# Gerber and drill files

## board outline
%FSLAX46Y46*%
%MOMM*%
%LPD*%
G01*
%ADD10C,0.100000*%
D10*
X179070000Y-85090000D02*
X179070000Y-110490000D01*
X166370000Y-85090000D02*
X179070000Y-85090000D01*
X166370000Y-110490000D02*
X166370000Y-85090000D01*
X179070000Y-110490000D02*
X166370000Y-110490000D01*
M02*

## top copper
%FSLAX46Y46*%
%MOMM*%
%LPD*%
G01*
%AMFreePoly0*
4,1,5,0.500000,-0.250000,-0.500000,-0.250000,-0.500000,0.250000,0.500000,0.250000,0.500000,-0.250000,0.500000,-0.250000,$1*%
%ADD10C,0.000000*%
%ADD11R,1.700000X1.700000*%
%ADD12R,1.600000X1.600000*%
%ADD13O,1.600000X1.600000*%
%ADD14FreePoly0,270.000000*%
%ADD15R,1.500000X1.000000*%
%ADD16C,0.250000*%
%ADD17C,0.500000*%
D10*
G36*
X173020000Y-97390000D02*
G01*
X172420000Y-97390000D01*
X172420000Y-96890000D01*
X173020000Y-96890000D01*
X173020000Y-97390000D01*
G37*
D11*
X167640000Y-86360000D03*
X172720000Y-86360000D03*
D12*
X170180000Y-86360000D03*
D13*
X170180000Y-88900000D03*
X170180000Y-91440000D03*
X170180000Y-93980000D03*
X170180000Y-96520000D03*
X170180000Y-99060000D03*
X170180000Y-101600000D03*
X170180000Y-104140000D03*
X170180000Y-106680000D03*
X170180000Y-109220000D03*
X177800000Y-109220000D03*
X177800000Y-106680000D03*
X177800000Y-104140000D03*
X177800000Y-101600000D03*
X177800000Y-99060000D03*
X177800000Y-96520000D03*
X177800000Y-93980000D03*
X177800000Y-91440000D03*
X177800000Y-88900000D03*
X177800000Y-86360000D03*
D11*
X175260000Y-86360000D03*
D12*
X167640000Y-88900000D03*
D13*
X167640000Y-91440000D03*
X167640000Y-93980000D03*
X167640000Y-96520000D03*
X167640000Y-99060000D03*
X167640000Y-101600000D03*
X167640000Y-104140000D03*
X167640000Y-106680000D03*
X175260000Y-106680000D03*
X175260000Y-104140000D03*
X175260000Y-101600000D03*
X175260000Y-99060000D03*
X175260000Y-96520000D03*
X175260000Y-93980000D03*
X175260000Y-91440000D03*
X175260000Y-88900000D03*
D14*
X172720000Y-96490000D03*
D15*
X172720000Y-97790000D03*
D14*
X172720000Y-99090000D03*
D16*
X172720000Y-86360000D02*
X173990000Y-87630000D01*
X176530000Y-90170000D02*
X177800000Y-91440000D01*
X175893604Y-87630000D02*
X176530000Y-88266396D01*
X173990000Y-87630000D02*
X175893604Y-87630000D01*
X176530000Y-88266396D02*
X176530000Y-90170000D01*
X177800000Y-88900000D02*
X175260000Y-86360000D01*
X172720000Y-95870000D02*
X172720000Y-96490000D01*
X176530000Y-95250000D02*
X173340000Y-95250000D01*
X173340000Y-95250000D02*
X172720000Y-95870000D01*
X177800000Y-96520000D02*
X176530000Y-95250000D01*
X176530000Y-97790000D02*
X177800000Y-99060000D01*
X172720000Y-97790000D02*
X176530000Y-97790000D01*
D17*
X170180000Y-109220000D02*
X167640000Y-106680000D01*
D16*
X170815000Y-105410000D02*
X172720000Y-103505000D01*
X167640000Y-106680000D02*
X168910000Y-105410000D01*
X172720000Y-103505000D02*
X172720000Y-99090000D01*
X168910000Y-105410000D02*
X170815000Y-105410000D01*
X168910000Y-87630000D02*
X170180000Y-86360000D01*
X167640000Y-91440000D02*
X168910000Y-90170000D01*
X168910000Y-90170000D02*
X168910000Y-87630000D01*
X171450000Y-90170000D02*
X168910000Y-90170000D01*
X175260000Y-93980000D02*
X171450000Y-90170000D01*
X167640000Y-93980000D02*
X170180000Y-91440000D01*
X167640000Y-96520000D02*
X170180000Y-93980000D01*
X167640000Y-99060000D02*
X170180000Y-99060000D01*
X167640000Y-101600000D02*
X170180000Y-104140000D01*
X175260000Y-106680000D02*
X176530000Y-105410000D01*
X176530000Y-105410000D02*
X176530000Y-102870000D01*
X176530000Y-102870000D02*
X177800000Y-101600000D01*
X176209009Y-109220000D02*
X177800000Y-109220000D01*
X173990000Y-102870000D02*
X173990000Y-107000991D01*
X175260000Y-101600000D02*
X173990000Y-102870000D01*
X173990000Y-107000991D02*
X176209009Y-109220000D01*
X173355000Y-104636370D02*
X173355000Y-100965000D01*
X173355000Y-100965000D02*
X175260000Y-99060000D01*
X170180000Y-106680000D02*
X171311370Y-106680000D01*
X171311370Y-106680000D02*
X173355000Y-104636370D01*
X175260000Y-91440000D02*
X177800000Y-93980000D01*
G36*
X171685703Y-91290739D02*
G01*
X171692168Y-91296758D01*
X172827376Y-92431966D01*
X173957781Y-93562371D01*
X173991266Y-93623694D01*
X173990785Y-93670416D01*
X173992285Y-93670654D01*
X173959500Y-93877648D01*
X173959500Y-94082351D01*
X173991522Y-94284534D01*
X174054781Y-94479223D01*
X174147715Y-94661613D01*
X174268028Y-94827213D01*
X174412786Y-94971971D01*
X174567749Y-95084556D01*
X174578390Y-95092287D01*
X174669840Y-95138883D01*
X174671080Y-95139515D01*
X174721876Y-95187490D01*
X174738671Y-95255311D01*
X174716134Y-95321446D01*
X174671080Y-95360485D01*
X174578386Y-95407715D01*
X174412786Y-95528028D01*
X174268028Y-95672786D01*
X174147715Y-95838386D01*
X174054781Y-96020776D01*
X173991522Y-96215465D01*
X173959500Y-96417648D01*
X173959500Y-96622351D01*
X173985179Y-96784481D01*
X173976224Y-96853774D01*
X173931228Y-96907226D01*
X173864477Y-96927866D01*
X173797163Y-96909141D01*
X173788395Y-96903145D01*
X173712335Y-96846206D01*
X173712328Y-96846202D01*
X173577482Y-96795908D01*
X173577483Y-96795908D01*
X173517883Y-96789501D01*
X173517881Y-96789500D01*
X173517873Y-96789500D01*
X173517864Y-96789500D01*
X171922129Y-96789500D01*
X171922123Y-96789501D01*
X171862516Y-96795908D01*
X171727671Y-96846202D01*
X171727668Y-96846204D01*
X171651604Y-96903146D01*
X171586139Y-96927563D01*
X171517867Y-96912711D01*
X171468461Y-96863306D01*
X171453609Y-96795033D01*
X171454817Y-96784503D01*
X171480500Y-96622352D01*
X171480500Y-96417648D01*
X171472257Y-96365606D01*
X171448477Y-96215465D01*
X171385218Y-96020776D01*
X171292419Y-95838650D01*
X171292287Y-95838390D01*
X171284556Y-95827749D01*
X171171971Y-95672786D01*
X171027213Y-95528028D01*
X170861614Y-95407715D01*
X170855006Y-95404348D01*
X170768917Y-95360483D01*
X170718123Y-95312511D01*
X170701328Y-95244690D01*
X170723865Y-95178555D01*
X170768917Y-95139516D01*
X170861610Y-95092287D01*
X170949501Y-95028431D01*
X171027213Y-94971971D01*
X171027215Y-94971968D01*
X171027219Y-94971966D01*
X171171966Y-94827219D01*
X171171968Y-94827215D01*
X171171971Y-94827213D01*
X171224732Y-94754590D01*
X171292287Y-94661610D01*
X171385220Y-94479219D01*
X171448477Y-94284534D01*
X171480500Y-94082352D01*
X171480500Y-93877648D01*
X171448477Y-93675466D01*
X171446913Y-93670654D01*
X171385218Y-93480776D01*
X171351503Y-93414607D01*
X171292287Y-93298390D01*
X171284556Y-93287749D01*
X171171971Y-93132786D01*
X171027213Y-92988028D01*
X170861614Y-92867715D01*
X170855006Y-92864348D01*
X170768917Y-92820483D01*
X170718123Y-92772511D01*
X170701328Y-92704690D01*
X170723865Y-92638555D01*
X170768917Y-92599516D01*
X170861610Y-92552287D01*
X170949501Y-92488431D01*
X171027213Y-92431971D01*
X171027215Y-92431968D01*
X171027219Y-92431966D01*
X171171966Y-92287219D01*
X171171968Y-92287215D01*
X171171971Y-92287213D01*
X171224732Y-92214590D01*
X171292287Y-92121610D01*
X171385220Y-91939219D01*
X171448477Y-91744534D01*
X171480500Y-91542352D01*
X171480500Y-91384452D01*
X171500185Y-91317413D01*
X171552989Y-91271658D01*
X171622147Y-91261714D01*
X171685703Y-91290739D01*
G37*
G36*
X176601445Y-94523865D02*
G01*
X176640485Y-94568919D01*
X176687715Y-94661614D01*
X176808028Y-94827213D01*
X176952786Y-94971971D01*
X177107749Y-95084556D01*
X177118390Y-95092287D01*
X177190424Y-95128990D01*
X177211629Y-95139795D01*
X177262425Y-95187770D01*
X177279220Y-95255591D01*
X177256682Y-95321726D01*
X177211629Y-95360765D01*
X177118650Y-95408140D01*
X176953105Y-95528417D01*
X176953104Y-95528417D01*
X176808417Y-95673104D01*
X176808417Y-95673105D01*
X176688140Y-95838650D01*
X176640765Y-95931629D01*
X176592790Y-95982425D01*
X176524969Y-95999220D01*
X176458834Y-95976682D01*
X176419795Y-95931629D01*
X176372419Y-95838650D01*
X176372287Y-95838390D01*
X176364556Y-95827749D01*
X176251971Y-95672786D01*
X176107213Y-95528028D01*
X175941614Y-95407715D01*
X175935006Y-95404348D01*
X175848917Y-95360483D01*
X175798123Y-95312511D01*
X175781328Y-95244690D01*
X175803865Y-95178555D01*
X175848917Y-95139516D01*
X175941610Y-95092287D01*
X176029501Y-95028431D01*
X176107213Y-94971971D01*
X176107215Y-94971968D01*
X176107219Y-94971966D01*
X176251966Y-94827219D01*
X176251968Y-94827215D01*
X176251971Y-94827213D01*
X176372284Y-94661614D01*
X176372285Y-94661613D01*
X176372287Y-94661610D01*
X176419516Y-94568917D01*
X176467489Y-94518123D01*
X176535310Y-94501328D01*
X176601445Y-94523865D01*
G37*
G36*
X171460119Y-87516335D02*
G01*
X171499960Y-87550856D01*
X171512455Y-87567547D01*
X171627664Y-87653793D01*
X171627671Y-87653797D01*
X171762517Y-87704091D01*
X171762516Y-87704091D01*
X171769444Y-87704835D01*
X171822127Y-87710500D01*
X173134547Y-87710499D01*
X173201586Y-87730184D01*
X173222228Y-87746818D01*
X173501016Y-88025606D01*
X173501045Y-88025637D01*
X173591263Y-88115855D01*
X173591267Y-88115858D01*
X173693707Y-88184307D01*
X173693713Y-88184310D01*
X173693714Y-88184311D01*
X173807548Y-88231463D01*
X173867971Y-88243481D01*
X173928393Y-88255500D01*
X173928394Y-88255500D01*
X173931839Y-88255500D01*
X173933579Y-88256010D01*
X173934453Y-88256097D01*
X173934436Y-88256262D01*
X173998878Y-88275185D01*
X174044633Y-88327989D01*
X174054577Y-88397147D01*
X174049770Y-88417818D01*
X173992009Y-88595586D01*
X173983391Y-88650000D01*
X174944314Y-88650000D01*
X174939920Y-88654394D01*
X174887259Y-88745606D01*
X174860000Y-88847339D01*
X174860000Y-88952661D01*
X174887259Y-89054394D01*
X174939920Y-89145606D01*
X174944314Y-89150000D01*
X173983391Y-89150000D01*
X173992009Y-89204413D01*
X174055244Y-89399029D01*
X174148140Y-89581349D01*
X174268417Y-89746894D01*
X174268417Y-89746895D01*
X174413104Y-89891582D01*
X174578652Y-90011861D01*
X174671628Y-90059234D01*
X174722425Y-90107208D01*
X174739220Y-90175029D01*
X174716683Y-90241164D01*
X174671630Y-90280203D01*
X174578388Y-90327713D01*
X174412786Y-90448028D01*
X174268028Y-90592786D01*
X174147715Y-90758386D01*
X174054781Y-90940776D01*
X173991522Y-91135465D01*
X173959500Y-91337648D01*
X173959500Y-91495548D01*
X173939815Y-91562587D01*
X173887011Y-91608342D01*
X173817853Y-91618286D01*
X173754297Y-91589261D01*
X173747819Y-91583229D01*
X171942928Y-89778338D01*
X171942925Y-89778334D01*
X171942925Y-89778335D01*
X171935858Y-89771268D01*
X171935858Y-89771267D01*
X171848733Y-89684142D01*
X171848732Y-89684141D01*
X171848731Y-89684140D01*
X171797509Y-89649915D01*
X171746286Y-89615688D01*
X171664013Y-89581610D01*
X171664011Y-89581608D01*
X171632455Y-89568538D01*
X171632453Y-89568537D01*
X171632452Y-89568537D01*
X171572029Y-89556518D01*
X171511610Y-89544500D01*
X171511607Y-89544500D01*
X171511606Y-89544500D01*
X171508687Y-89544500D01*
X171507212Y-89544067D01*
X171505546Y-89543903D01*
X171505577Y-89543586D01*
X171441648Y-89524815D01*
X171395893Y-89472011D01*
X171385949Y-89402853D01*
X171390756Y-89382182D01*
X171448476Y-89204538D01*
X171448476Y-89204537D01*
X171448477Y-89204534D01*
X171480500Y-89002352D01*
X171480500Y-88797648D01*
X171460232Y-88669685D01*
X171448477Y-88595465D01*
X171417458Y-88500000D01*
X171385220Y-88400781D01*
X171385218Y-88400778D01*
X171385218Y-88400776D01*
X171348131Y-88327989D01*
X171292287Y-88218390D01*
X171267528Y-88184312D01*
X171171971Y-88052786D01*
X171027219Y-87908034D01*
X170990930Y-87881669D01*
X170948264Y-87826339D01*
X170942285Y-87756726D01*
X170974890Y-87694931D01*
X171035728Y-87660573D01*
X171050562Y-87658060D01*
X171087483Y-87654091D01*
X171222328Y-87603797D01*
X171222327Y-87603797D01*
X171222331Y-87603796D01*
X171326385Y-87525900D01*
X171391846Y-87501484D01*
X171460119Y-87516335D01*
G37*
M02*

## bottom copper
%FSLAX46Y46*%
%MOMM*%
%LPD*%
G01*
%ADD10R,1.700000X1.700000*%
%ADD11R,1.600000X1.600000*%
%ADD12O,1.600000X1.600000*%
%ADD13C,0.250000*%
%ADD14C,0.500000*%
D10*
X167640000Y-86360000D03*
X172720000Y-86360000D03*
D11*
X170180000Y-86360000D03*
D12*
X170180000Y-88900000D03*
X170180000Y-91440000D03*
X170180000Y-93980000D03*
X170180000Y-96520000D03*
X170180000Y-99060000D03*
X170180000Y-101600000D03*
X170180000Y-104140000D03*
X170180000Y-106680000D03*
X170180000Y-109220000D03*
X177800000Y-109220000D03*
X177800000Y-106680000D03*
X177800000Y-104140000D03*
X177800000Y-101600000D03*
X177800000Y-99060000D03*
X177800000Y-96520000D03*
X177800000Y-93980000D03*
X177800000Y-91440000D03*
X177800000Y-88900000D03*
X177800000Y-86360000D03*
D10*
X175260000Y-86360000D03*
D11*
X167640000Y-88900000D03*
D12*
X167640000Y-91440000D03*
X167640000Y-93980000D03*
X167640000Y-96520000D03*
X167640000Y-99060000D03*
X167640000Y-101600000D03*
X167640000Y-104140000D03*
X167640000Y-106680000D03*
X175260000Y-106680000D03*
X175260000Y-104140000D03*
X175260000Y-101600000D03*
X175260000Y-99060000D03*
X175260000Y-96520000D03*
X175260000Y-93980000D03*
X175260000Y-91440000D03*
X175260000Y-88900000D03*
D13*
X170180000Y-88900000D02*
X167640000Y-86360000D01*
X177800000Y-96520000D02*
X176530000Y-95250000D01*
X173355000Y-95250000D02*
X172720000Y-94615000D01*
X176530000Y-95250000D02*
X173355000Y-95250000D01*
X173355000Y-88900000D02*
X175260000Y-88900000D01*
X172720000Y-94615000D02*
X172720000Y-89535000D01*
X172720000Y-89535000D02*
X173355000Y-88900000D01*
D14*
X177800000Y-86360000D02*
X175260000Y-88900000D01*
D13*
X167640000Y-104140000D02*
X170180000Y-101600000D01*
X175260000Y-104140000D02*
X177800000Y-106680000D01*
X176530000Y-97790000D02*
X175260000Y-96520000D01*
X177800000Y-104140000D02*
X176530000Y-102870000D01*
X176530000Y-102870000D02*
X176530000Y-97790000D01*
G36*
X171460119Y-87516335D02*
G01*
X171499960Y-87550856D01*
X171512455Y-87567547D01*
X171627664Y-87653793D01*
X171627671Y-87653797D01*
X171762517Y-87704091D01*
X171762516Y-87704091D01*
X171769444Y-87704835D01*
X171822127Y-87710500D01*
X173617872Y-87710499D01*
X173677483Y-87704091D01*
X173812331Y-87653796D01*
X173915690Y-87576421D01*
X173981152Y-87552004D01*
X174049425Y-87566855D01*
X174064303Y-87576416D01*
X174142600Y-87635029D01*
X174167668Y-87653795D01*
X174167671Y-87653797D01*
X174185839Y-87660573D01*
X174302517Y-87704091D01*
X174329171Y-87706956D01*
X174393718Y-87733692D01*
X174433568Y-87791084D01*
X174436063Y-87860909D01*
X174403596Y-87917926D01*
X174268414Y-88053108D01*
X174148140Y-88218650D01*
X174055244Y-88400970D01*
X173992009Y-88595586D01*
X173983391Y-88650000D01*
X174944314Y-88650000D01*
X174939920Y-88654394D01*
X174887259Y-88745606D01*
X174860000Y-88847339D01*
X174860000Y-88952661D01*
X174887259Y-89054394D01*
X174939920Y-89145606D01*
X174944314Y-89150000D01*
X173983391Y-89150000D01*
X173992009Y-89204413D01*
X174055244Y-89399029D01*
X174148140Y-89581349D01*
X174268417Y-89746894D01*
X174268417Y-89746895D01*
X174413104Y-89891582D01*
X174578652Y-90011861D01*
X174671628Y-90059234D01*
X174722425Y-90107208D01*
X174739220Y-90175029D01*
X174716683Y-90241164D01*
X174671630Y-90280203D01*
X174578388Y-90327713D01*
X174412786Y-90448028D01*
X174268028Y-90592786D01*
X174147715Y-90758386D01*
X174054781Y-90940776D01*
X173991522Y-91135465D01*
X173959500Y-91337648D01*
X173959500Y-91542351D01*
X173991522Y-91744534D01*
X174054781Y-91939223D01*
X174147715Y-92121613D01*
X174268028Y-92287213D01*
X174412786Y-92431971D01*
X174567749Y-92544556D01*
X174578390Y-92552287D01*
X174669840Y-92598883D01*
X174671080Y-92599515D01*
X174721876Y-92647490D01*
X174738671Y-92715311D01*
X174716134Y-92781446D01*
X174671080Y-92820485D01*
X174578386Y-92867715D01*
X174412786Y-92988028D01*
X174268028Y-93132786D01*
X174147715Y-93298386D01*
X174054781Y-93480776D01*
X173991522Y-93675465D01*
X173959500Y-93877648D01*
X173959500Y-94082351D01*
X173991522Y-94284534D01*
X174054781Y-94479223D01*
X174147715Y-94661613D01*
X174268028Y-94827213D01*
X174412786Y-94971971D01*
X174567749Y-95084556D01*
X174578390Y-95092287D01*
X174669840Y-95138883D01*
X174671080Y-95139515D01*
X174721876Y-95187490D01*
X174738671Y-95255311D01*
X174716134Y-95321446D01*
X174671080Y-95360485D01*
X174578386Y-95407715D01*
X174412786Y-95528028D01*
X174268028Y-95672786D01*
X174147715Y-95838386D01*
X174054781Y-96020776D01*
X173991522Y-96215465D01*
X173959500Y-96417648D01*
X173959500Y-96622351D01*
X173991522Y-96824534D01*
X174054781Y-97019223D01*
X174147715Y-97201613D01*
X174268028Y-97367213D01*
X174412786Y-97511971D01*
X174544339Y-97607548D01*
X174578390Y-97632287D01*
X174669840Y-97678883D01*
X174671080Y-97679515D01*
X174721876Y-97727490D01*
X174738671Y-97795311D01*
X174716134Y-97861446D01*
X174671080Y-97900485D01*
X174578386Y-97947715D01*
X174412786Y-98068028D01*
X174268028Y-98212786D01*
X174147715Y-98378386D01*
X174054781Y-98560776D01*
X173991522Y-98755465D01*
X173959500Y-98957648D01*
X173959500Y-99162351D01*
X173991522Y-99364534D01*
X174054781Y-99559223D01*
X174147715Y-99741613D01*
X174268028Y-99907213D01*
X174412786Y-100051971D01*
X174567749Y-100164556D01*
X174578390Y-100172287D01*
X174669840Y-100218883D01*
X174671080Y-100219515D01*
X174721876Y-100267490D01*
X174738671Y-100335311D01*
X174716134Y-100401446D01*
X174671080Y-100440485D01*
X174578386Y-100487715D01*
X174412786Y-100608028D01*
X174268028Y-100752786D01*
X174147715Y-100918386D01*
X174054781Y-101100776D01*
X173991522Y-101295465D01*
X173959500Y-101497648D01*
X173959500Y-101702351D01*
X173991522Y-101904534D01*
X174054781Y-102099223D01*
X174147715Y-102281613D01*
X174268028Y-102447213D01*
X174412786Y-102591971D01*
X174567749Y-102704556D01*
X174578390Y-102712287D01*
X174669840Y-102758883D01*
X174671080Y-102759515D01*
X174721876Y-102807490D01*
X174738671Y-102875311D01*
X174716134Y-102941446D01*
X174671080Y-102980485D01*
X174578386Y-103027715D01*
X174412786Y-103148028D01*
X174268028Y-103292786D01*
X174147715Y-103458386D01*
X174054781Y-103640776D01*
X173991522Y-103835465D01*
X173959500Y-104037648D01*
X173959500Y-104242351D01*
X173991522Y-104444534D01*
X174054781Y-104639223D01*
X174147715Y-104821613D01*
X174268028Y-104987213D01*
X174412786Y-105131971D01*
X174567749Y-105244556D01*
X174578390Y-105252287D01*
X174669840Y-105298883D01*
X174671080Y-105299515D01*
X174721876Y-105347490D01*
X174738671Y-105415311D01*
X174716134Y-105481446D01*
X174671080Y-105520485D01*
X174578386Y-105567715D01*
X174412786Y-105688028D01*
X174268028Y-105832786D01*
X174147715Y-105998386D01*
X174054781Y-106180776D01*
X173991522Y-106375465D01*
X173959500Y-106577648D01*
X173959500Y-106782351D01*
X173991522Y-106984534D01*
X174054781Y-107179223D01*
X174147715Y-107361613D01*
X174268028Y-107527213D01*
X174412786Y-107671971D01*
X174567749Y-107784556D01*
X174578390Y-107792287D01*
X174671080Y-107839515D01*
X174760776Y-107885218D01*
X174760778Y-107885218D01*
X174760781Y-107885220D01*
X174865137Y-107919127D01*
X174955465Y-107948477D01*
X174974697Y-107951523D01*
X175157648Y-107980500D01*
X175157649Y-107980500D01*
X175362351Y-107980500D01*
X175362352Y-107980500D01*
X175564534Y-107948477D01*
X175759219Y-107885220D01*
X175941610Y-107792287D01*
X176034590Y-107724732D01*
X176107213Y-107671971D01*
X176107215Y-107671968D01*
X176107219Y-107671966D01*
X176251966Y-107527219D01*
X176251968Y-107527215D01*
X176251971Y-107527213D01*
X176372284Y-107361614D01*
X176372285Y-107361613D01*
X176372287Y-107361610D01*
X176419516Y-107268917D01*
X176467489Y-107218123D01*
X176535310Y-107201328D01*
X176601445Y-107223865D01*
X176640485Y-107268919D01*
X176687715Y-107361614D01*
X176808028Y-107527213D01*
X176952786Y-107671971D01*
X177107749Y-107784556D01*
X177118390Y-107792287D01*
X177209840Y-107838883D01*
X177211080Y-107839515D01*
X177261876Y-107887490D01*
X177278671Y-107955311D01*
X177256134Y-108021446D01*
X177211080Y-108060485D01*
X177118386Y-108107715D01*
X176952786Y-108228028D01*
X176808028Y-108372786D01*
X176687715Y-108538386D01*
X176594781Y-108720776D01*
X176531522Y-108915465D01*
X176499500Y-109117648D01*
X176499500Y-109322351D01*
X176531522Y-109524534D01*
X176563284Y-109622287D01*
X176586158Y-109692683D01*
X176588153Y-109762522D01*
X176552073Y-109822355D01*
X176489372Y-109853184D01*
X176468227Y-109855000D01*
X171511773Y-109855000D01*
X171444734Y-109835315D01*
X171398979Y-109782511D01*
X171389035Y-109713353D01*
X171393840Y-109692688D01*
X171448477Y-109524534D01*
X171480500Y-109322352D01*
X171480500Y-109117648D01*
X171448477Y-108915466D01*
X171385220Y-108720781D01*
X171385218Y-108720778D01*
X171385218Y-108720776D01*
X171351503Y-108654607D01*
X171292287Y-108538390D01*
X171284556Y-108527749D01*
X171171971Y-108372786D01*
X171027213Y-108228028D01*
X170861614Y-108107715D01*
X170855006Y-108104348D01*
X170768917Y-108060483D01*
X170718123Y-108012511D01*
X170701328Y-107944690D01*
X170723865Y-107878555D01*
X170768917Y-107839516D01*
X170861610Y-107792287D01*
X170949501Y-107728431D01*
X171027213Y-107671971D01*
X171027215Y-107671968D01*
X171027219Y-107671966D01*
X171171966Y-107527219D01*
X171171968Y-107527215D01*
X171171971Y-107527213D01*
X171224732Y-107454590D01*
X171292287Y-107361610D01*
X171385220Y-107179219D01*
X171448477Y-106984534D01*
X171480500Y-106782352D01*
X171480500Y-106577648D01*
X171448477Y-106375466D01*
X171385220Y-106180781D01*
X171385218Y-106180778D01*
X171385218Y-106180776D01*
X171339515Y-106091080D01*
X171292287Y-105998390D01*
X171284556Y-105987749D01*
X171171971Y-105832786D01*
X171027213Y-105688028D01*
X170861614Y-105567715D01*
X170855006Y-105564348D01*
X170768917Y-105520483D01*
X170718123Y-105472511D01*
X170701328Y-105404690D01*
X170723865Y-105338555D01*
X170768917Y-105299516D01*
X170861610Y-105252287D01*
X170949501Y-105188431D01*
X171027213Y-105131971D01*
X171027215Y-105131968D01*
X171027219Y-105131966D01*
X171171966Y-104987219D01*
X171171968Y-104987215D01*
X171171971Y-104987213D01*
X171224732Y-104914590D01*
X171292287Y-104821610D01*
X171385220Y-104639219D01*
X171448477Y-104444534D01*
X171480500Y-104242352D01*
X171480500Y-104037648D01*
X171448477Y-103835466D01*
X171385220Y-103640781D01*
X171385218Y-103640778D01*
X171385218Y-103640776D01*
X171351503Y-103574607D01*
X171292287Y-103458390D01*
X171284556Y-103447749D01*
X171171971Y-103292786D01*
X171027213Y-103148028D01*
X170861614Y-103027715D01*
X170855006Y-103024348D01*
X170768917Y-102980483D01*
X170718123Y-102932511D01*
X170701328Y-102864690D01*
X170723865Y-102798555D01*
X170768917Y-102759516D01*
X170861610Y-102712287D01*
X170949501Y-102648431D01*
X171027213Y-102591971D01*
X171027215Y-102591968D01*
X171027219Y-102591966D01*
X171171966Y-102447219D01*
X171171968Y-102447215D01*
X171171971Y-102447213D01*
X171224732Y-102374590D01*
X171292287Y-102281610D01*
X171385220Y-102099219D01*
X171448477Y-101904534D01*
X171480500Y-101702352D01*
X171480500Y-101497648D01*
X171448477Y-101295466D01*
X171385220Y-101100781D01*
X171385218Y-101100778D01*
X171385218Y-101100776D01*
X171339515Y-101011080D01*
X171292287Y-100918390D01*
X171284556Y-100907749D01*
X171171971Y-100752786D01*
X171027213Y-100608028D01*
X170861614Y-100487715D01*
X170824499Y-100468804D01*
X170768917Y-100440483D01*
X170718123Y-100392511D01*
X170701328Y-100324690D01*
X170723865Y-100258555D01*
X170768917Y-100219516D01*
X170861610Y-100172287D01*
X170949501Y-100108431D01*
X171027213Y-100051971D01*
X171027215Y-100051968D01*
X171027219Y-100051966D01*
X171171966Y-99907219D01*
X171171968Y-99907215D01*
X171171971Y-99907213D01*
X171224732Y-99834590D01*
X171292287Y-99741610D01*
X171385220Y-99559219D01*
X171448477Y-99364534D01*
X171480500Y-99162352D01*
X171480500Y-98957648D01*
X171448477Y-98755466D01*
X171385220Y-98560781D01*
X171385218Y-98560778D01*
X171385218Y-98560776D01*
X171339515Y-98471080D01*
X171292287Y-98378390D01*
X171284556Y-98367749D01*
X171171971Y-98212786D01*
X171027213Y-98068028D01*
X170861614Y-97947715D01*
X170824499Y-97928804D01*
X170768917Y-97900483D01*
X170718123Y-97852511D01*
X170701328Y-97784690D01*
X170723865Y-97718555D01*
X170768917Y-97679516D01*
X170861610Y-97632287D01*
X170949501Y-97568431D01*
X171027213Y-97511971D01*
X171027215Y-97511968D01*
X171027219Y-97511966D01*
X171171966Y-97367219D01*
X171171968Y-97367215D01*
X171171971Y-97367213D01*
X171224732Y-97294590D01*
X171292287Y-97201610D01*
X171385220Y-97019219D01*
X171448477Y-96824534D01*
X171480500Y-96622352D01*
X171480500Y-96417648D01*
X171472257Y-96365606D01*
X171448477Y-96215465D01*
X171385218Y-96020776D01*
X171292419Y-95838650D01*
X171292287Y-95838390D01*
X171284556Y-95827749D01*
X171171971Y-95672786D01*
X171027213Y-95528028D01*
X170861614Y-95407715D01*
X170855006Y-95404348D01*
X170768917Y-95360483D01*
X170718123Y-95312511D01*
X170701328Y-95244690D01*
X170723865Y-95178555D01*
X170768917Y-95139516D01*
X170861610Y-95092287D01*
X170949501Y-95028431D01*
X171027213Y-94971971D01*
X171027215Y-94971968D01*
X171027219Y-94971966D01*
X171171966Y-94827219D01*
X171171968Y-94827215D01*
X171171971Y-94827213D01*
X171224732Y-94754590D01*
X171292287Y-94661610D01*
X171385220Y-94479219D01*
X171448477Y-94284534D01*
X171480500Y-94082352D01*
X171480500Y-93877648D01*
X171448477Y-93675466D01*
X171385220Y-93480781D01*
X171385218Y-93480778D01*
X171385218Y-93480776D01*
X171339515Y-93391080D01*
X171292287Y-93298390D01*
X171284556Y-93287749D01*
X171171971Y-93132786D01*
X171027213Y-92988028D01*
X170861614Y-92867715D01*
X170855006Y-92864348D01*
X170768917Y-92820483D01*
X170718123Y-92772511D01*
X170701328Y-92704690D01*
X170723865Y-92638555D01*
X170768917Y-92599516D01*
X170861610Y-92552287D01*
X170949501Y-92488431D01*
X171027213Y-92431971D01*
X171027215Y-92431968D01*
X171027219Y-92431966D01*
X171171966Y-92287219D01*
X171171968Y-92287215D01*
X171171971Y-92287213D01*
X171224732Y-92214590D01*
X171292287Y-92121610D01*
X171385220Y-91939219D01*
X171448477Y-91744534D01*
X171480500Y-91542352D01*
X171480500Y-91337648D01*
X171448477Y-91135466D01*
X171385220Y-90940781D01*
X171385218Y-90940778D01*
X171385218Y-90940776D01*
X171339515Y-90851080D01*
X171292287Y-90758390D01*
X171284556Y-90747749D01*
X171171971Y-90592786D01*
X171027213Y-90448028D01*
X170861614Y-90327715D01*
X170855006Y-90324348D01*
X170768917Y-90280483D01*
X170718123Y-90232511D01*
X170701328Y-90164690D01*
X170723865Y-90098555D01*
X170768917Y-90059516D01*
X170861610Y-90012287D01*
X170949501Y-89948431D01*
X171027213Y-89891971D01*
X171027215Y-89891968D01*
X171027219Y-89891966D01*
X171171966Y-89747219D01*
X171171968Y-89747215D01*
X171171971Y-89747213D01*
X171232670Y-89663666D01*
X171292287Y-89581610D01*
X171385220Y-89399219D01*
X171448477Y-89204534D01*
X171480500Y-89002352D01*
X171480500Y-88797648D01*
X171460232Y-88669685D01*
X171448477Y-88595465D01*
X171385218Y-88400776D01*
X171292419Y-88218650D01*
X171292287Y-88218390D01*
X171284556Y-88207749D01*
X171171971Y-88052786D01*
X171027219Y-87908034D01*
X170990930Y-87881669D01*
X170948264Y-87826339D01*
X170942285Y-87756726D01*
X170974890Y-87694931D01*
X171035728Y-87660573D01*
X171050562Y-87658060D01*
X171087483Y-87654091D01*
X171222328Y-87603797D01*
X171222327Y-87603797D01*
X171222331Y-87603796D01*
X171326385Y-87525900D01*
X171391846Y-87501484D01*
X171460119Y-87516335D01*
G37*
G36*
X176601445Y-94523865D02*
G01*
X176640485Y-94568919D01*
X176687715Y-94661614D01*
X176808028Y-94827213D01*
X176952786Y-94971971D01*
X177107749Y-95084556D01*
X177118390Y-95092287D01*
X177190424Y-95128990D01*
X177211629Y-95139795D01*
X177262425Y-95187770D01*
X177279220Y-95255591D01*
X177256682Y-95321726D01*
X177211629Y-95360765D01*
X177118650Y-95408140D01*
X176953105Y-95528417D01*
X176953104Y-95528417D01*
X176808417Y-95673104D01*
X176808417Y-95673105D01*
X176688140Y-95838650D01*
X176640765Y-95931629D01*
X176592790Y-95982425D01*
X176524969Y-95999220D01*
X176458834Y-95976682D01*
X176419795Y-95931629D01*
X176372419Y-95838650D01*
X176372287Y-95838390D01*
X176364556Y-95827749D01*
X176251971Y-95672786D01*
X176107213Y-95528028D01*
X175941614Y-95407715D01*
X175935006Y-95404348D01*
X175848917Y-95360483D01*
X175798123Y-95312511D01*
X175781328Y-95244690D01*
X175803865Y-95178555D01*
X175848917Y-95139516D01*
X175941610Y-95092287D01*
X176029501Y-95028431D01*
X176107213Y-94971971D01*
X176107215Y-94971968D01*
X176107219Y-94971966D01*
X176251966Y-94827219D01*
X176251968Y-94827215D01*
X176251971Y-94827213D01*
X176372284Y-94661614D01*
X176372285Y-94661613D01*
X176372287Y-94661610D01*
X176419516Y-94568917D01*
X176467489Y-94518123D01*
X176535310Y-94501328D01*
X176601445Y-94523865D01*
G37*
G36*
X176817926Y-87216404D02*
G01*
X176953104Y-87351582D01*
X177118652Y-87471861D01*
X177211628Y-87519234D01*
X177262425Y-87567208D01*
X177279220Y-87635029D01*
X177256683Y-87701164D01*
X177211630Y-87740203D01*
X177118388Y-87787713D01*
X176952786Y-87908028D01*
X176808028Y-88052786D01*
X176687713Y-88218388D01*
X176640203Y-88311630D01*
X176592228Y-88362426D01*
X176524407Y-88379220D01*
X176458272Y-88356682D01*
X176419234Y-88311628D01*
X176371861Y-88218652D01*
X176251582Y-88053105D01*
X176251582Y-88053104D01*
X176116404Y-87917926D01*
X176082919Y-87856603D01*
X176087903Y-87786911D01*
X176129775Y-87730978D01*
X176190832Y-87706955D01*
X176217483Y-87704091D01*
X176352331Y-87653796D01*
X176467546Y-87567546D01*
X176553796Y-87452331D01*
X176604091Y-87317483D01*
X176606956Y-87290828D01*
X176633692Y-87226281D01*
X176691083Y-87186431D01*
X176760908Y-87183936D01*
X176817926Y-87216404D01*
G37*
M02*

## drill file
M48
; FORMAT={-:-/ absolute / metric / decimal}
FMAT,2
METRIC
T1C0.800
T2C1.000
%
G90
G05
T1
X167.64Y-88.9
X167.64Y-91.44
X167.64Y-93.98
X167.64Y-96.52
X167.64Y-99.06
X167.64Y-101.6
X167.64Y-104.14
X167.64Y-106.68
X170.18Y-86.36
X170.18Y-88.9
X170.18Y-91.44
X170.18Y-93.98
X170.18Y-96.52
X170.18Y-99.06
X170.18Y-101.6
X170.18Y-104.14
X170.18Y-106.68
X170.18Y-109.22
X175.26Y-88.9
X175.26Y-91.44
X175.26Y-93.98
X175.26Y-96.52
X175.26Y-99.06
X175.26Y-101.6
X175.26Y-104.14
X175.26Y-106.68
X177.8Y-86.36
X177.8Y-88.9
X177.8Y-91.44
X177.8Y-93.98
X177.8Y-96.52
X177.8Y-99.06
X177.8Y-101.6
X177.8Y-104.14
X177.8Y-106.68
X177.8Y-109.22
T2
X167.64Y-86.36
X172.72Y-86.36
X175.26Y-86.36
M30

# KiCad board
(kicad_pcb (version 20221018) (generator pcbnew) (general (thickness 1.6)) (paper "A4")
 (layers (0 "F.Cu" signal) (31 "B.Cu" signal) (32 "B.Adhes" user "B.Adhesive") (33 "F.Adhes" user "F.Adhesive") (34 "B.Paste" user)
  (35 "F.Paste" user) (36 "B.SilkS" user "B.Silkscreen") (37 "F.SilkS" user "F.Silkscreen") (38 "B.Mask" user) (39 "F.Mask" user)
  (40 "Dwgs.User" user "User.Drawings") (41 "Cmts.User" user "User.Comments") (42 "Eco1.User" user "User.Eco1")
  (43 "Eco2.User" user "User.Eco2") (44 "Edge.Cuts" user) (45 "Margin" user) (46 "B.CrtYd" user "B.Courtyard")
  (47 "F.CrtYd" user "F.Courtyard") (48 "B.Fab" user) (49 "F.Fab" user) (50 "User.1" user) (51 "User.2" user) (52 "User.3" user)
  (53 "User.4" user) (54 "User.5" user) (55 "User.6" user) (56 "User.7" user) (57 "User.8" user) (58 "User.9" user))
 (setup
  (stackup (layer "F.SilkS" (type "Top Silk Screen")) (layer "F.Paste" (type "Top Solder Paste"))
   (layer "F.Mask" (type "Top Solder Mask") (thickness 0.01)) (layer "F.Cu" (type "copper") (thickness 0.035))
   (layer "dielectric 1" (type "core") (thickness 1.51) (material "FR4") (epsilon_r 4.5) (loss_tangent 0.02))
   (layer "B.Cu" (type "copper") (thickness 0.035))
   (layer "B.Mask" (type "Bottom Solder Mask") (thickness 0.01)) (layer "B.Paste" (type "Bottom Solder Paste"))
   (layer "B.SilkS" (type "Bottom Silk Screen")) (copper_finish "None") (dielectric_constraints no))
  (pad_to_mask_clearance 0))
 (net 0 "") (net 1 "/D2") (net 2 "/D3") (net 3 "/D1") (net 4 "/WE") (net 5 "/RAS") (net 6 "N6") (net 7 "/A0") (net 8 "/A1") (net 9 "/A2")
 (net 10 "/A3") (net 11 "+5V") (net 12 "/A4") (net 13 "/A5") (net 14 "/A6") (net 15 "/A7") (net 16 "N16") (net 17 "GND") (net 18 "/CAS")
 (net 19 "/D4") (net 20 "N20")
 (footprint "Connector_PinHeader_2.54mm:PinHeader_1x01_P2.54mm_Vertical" (layer "F.Cu") (at 167.64 86.36)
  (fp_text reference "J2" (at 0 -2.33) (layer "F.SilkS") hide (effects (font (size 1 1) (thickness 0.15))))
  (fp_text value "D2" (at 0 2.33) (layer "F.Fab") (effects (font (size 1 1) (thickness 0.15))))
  (pad "1" thru_hole rect (at 0 0) (size 1.7 1.7) (drill 1) (layers "*.Cu" "*.Mask") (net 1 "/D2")))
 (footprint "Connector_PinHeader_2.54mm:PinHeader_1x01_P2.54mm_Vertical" (layer "F.Cu") (at 172.72 86.36)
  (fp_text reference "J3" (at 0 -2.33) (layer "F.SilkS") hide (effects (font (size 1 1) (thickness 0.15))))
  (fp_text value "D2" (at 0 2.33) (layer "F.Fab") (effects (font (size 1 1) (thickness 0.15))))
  (pad "1" thru_hole rect (at 0 0) (size 1.7 1.7) (drill 1) (layers "*.Cu" "*.Mask") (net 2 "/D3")))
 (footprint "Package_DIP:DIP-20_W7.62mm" (layer "F.Cu") (at 170.18 86.36)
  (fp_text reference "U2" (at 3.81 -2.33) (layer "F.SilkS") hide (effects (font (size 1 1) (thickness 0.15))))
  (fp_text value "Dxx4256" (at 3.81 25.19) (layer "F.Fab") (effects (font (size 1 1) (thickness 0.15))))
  (pad "1" thru_hole rect (at 0 0) (size 1.6 1.6) (drill 0.8) (layers "*.Cu" "*.Mask") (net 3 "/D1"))
  (pad "2" thru_hole oval (at 0 2.54) (size 1.6 1.6) (drill 0.8) (layers "*.Cu" "*.Mask") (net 1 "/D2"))
  (pad "3" thru_hole oval (at 0 5.08) (size 1.6 1.6) (drill 0.8) (layers "*.Cu" "*.Mask") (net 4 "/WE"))
  (pad "4" thru_hole oval (at 0 7.62) (size 1.6 1.6) (drill 0.8) (layers "*.Cu" "*.Mask") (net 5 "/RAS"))
  (pad "5" thru_hole oval (at 0 10.16) (size 1.6 1.6) (drill 0.8) (layers "*.Cu" "*.Mask") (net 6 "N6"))
  (pad "6" thru_hole oval (at 0 12.7) (size 1.6 1.6) (drill 0.8) (layers "*.Cu" "*.Mask") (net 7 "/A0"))
  (pad "7" thru_hole oval (at 0 15.24) (size 1.6 1.6) (drill 0.8) (layers "*.Cu" "*.Mask") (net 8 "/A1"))
  (pad "8" thru_hole oval (at 0 17.78) (size 1.6 1.6) (drill 0.8) (layers "*.Cu" "*.Mask") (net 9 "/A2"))
  (pad "9" thru_hole oval (at 0 20.32) (size 1.6 1.6) (drill 0.8) (layers "*.Cu" "*.Mask") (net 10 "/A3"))
  (pad "10" thru_hole oval (at 0 22.86) (size 1.6 1.6) (drill 0.8) (layers "*.Cu" "*.Mask") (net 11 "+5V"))
  (pad "11" thru_hole oval (at 7.62 22.86) (size 1.6 1.6) (drill 0.8) (layers "*.Cu" "*.Mask") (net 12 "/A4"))
  (pad "12" thru_hole oval (at 7.62 20.32) (size 1.6 1.6) (drill 0.8) (layers "*.Cu" "*.Mask") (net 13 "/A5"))
  (pad "13" thru_hole oval (at 7.62 17.78) (size 1.6 1.6) (drill 0.8) (layers "*.Cu" "*.Mask") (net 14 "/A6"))
  (pad "14" thru_hole oval (at 7.62 15.24) (size 1.6 1.6) (drill 0.8) (layers "*.Cu" "*.Mask") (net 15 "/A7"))
  (pad "15" thru_hole oval (at 7.62 12.7) (size 1.6 1.6) (drill 0.8) (layers "*.Cu" "*.Mask") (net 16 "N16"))
  (pad "16" thru_hole oval (at 7.62 10.16) (size 1.6 1.6) (drill 0.8) (layers "*.Cu" "*.Mask") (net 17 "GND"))
  (pad "17" thru_hole oval (at 7.62 7.62) (size 1.6 1.6) (drill 0.8) (layers "*.Cu" "*.Mask") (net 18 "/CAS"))
  (pad "18" thru_hole oval (at 7.62 5.08) (size 1.6 1.6) (drill 0.8) (layers "*.Cu" "*.Mask") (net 2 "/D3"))
  (pad "19" thru_hole oval (at 7.62 2.54) (size 1.6 1.6) (drill 0.8) (layers "*.Cu" "*.Mask") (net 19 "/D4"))
  (pad "20" thru_hole oval (at 7.62 0) (size 1.6 1.6) (drill 0.8) (layers "*.Cu" "*.Mask") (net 17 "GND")))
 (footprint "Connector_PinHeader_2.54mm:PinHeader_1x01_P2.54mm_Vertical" (layer "F.Cu") (at 175.26 86.36)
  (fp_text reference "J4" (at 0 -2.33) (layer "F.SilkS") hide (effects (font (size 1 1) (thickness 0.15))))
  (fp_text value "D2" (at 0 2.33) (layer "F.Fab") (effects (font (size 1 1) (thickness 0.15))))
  (pad "1" thru_hole rect (at 0 0) (size 1.7 1.7) (drill 1) (layers "*.Cu" "*.Mask") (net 19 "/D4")))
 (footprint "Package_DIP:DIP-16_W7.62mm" (layer "F.Cu") (at 167.64 88.9)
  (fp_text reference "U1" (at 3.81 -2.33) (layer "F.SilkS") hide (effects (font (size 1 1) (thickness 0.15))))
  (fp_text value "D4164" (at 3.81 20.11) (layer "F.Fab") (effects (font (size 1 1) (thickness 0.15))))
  (pad "1" thru_hole rect (at 0 0) (size 1.6 1.6) (drill 0.8) (layers "*.Cu" "*.Mask") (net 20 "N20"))
  (pad "2" thru_hole oval (at 0 2.54) (size 1.6 1.6) (drill 0.8) (layers "*.Cu" "*.Mask") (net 3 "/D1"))
  (pad "3" thru_hole oval (at 0 5.08) (size 1.6 1.6) (drill 0.8) (layers "*.Cu" "*.Mask") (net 4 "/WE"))
  (pad "4" thru_hole oval (at 0 7.62) (size 1.6 1.6) (drill 0.8) (layers "*.Cu" "*.Mask") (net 5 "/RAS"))
  (pad "5" thru_hole oval (at 0 10.16) (size 1.6 1.6) (drill 0.8) (layers "*.Cu" "*.Mask") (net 7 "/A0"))
  (pad "6" thru_hole oval (at 0 12.7) (size 1.6 1.6) (drill 0.8) (layers "*.Cu" "*.Mask") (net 9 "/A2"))
  (pad "7" thru_hole oval (at 0 15.24) (size 1.6 1.6) (drill 0.8) (layers "*.Cu" "*.Mask") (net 8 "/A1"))
  (pad "8" thru_hole oval (at 0 17.78) (size 1.6 1.6) (drill 0.8) (layers "*.Cu" "*.Mask") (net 11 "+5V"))
  (pad "9" thru_hole oval (at 7.62 17.78) (size 1.6 1.6) (drill 0.8) (layers "*.Cu" "*.Mask") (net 15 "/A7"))
  (pad "10" thru_hole oval (at 7.62 15.24) (size 1.6 1.6) (drill 0.8) (layers "*.Cu" "*.Mask") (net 13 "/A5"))
  (pad "11" thru_hole oval (at 7.62 12.7) (size 1.6 1.6) (drill 0.8) (layers "*.Cu" "*.Mask") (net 12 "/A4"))
  (pad "12" thru_hole oval (at 7.62 10.16) (size 1.6 1.6) (drill 0.8) (layers "*.Cu" "*.Mask") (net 10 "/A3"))
  (pad "13" thru_hole oval (at 7.62 7.62) (size 1.6 1.6) (drill 0.8) (layers "*.Cu" "*.Mask") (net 14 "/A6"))
  (pad "14" thru_hole oval (at 7.62 5.08) (size 1.6 1.6) (drill 0.8) (layers "*.Cu" "*.Mask") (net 3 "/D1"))
  (pad "15" thru_hole oval (at 7.62 2.54) (size 1.6 1.6) (drill 0.8) (layers "*.Cu" "*.Mask") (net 18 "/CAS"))
  (pad "16" thru_hole oval (at 7.62 0) (size 1.6 1.6) (drill 0.8) (layers "*.Cu" "*.Mask") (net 17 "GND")))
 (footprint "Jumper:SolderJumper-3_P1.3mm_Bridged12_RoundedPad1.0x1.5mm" (layer "F.Cu") (at 172.72 97.79 -90) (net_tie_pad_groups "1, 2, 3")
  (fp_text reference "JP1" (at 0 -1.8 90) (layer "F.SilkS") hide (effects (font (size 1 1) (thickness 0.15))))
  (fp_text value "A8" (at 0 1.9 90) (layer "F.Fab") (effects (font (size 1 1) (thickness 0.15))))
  (fp_poly (pts (xy -0.9 -0.3) (xy -0.4 -0.3) (xy -0.4 0.3) (xy -0.9 0.3)) (stroke (width 0) (type solid)) (fill solid) (layer "F.Cu"))
  (pad "1" smd custom (at -1.3 0 270) (size 1 0.5) (layers "F.Cu" "F.Mask") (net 17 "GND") (zone_connect 2) (thermal_bridge_angle 45)
   (options (clearance outline) (anchor rect)) (primitives))
  (pad "2" smd rect (at 0 0 270) (size 1 1.5) (layers "F.Cu" "F.Mask") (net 16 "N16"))
  (pad "3" smd custom (at 1.3 0 270) (size 1 0.5) (layers "F.Cu" "F.Mask") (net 11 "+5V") (zone_connect 2) (thermal_bridge_angle 45)
   (options (clearance outline) (anchor rect)) (primitives)))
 (gr_line (start 179.07 85.09) (end 179.07 110.49) (stroke (width 0.1) (type default)) (layer "Edge.Cuts"))
 (gr_line (start 166.37 85.09) (end 179.07 85.09) (stroke (width 0.1) (type default)) (layer "Edge.Cuts"))
 (gr_line (start 166.37 110.49) (end 166.37 85.09) (stroke (width 0.1) (type default)) (layer "Edge.Cuts"))
 (gr_line (start 179.07 110.49) (end 166.37 110.49) (stroke (width 0.1) (type default)) (layer "Edge.Cuts"))
 (segment (start 170.18 88.9) (end 167.64 86.36) (width 0.25) (layer "B.Cu") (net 1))
 (segment (start 172.72 86.36) (end 173.99 87.63) (width 0.25) (layer "F.Cu") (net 2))
 (segment (start 176.53 90.17) (end 177.8 91.44) (width 0.25) (layer "F.Cu") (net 2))
 (segment (start 175.893604 87.63) (end 176.53 88.266396) (width 0.25) (layer "F.Cu") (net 2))
 (segment (start 173.99 87.63) (end 175.893604 87.63) (width 0.25) (layer "F.Cu") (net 2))
 (segment (start 176.53 88.266396) (end 176.53 90.17) (width 0.25) (layer "F.Cu") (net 2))
 (segment (start 177.8 88.9) (end 175.26 86.36) (width 0.25) (layer "F.Cu") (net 19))
 (segment (start 172.72 95.87) (end 172.72 96.49) (width 0.25) (layer "F.Cu") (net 17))
 (segment (start 176.53 95.25) (end 173.34 95.25) (width 0.25) (layer "F.Cu") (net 17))
 (segment (start 173.34 95.25) (end 172.72 95.87) (width 0.25) (layer "F.Cu") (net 17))
 (segment (start 177.8 96.52) (end 176.53 95.25) (width 0.25) (layer "F.Cu") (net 17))
 (segment (start 177.8 96.52) (end 176.53 95.25) (width 0.25) (layer "B.Cu") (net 17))
 (segment (start 173.355 95.25) (end 172.72 94.615) (width 0.25) (layer "B.Cu") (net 17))
 (segment (start 176.53 95.25) (end 173.355 95.25) (width 0.25) (layer "B.Cu") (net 17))
 (segment (start 173.355 88.9) (end 175.26 88.9) (width 0.25) (layer "B.Cu") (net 17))
 (segment (start 172.72 94.615) (end 172.72 89.535) (width 0.25) (layer "B.Cu") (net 17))
 (segment (start 172.72 89.535) (end 173.355 88.9) (width 0.25) (layer "B.Cu") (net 17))
 (segment (start 177.8 86.36) (end 175.26 88.9) (width 0.5) (layer "B.Cu") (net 17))
 (segment (start 176.53 97.79) (end 177.8 99.06) (width 0.25) (layer "F.Cu") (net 16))
 (segment (start 172.72 97.79) (end 176.53 97.79) (width 0.25) (layer "F.Cu") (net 16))
 (segment (start 170.18 109.22) (end 167.64 106.68) (width 0.5) (layer "F.Cu") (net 11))
 (segment (start 170.815 105.41) (end 172.72 103.505) (width 0.25) (layer "F.Cu") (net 11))
 (segment (start 167.64 106.68) (end 168.91 105.41) (width 0.25) (layer "F.Cu") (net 11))
 (segment (start 172.72 103.505) (end 172.72 99.09) (width 0.25) (layer "F.Cu") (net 11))
 (segment (start 168.91 105.41) (end 170.815 105.41) (width 0.25) (layer "F.Cu") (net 11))
 (segment (start 168.91 87.63) (end 170.18 86.36) (width 0.25) (layer "F.Cu") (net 3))
 (segment (start 167.64 91.44) (end 168.91 90.17) (width 0.25) (layer "F.Cu") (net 3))
 (segment (start 168.91 90.17) (end 168.91 87.63) (width 0.25) (layer "F.Cu") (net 3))
 (segment (start 171.45 90.17) (end 168.91 90.17) (width 0.25) (layer "F.Cu") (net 3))
 (segment (start 175.26 93.98) (end 171.45 90.17) (width 0.25) (layer "F.Cu") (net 3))
 (segment (start 167.64 93.98) (end 170.18 91.44) (width 0.25) (layer "F.Cu") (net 4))
 (segment (start 167.64 96.52) (end 170.18 93.98) (width 0.25) (layer "F.Cu") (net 5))
 (segment (start 167.64 99.06) (end 170.18 99.06) (width 0.25) (layer "F.Cu") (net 7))
 (segment (start 167.64 101.6) (end 170.18 104.14) (width 0.25) (layer "F.Cu") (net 9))
 (segment (start 167.64 104.14) (end 170.18 101.6) (width 0.25) (layer "B.Cu") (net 8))
 (segment (start 175.26 106.68) (end 176.53 105.41) (width 0.25) (layer "F.Cu") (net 15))
 (segment (start 176.53 105.41) (end 176.53 102.87) (width 0.25) (layer "F.Cu") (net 15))
 (segment (start 176.53 102.87) (end 177.8 101.6) (width 0.25) (layer "F.Cu") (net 15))
 (segment (start 175.26 104.14) (end 177.8 106.68) (width 0.25) (layer "B.Cu") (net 13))
 (segment (start 176.209009 109.22) (end 177.8 109.22) (width 0.25) (layer "F.Cu") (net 12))
 (segment (start 173.99 102.87) (end 173.99 107.000991) (width 0.25) (layer "F.Cu") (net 12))
 (segment (start 175.26 101.6) (end 173.99 102.87) (width 0.25) (layer "F.Cu") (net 12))
 (segment (start 173.99 107.000991) (end 176.209009 109.22) (width 0.25) (layer "F.Cu") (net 12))
 (segment (start 173.355 104.63637) (end 173.355 100.965) (width 0.25) (layer "F.Cu") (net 10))
 (segment (start 173.355 100.965) (end 175.26 99.06) (width 0.25) (layer "F.Cu") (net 10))
 (segment (start 170.18 106.68) (end 171.31137 106.68) (width 0.25) (layer "F.Cu") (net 10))
 (segment (start 171.31137 106.68) (end 173.355 104.63637) (width 0.25) (layer "F.Cu") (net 10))
 (segment (start 176.53 97.79) (end 175.26 96.52) (width 0.25) (layer "B.Cu") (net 14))
 (segment (start 177.8 104.14) (end 176.53 102.87) (width 0.25) (layer "B.Cu") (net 14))
 (segment (start 176.53 102.87) (end 176.53 97.79) (width 0.25) (layer "B.Cu") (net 14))
 (segment (start 175.26 91.44) (end 177.8 93.98) (width 0.25) (layer "F.Cu") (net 18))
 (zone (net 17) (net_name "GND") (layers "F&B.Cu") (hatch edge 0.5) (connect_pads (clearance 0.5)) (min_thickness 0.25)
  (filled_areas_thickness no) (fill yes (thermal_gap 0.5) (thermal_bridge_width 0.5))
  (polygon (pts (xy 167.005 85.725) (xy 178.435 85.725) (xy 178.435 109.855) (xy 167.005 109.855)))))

